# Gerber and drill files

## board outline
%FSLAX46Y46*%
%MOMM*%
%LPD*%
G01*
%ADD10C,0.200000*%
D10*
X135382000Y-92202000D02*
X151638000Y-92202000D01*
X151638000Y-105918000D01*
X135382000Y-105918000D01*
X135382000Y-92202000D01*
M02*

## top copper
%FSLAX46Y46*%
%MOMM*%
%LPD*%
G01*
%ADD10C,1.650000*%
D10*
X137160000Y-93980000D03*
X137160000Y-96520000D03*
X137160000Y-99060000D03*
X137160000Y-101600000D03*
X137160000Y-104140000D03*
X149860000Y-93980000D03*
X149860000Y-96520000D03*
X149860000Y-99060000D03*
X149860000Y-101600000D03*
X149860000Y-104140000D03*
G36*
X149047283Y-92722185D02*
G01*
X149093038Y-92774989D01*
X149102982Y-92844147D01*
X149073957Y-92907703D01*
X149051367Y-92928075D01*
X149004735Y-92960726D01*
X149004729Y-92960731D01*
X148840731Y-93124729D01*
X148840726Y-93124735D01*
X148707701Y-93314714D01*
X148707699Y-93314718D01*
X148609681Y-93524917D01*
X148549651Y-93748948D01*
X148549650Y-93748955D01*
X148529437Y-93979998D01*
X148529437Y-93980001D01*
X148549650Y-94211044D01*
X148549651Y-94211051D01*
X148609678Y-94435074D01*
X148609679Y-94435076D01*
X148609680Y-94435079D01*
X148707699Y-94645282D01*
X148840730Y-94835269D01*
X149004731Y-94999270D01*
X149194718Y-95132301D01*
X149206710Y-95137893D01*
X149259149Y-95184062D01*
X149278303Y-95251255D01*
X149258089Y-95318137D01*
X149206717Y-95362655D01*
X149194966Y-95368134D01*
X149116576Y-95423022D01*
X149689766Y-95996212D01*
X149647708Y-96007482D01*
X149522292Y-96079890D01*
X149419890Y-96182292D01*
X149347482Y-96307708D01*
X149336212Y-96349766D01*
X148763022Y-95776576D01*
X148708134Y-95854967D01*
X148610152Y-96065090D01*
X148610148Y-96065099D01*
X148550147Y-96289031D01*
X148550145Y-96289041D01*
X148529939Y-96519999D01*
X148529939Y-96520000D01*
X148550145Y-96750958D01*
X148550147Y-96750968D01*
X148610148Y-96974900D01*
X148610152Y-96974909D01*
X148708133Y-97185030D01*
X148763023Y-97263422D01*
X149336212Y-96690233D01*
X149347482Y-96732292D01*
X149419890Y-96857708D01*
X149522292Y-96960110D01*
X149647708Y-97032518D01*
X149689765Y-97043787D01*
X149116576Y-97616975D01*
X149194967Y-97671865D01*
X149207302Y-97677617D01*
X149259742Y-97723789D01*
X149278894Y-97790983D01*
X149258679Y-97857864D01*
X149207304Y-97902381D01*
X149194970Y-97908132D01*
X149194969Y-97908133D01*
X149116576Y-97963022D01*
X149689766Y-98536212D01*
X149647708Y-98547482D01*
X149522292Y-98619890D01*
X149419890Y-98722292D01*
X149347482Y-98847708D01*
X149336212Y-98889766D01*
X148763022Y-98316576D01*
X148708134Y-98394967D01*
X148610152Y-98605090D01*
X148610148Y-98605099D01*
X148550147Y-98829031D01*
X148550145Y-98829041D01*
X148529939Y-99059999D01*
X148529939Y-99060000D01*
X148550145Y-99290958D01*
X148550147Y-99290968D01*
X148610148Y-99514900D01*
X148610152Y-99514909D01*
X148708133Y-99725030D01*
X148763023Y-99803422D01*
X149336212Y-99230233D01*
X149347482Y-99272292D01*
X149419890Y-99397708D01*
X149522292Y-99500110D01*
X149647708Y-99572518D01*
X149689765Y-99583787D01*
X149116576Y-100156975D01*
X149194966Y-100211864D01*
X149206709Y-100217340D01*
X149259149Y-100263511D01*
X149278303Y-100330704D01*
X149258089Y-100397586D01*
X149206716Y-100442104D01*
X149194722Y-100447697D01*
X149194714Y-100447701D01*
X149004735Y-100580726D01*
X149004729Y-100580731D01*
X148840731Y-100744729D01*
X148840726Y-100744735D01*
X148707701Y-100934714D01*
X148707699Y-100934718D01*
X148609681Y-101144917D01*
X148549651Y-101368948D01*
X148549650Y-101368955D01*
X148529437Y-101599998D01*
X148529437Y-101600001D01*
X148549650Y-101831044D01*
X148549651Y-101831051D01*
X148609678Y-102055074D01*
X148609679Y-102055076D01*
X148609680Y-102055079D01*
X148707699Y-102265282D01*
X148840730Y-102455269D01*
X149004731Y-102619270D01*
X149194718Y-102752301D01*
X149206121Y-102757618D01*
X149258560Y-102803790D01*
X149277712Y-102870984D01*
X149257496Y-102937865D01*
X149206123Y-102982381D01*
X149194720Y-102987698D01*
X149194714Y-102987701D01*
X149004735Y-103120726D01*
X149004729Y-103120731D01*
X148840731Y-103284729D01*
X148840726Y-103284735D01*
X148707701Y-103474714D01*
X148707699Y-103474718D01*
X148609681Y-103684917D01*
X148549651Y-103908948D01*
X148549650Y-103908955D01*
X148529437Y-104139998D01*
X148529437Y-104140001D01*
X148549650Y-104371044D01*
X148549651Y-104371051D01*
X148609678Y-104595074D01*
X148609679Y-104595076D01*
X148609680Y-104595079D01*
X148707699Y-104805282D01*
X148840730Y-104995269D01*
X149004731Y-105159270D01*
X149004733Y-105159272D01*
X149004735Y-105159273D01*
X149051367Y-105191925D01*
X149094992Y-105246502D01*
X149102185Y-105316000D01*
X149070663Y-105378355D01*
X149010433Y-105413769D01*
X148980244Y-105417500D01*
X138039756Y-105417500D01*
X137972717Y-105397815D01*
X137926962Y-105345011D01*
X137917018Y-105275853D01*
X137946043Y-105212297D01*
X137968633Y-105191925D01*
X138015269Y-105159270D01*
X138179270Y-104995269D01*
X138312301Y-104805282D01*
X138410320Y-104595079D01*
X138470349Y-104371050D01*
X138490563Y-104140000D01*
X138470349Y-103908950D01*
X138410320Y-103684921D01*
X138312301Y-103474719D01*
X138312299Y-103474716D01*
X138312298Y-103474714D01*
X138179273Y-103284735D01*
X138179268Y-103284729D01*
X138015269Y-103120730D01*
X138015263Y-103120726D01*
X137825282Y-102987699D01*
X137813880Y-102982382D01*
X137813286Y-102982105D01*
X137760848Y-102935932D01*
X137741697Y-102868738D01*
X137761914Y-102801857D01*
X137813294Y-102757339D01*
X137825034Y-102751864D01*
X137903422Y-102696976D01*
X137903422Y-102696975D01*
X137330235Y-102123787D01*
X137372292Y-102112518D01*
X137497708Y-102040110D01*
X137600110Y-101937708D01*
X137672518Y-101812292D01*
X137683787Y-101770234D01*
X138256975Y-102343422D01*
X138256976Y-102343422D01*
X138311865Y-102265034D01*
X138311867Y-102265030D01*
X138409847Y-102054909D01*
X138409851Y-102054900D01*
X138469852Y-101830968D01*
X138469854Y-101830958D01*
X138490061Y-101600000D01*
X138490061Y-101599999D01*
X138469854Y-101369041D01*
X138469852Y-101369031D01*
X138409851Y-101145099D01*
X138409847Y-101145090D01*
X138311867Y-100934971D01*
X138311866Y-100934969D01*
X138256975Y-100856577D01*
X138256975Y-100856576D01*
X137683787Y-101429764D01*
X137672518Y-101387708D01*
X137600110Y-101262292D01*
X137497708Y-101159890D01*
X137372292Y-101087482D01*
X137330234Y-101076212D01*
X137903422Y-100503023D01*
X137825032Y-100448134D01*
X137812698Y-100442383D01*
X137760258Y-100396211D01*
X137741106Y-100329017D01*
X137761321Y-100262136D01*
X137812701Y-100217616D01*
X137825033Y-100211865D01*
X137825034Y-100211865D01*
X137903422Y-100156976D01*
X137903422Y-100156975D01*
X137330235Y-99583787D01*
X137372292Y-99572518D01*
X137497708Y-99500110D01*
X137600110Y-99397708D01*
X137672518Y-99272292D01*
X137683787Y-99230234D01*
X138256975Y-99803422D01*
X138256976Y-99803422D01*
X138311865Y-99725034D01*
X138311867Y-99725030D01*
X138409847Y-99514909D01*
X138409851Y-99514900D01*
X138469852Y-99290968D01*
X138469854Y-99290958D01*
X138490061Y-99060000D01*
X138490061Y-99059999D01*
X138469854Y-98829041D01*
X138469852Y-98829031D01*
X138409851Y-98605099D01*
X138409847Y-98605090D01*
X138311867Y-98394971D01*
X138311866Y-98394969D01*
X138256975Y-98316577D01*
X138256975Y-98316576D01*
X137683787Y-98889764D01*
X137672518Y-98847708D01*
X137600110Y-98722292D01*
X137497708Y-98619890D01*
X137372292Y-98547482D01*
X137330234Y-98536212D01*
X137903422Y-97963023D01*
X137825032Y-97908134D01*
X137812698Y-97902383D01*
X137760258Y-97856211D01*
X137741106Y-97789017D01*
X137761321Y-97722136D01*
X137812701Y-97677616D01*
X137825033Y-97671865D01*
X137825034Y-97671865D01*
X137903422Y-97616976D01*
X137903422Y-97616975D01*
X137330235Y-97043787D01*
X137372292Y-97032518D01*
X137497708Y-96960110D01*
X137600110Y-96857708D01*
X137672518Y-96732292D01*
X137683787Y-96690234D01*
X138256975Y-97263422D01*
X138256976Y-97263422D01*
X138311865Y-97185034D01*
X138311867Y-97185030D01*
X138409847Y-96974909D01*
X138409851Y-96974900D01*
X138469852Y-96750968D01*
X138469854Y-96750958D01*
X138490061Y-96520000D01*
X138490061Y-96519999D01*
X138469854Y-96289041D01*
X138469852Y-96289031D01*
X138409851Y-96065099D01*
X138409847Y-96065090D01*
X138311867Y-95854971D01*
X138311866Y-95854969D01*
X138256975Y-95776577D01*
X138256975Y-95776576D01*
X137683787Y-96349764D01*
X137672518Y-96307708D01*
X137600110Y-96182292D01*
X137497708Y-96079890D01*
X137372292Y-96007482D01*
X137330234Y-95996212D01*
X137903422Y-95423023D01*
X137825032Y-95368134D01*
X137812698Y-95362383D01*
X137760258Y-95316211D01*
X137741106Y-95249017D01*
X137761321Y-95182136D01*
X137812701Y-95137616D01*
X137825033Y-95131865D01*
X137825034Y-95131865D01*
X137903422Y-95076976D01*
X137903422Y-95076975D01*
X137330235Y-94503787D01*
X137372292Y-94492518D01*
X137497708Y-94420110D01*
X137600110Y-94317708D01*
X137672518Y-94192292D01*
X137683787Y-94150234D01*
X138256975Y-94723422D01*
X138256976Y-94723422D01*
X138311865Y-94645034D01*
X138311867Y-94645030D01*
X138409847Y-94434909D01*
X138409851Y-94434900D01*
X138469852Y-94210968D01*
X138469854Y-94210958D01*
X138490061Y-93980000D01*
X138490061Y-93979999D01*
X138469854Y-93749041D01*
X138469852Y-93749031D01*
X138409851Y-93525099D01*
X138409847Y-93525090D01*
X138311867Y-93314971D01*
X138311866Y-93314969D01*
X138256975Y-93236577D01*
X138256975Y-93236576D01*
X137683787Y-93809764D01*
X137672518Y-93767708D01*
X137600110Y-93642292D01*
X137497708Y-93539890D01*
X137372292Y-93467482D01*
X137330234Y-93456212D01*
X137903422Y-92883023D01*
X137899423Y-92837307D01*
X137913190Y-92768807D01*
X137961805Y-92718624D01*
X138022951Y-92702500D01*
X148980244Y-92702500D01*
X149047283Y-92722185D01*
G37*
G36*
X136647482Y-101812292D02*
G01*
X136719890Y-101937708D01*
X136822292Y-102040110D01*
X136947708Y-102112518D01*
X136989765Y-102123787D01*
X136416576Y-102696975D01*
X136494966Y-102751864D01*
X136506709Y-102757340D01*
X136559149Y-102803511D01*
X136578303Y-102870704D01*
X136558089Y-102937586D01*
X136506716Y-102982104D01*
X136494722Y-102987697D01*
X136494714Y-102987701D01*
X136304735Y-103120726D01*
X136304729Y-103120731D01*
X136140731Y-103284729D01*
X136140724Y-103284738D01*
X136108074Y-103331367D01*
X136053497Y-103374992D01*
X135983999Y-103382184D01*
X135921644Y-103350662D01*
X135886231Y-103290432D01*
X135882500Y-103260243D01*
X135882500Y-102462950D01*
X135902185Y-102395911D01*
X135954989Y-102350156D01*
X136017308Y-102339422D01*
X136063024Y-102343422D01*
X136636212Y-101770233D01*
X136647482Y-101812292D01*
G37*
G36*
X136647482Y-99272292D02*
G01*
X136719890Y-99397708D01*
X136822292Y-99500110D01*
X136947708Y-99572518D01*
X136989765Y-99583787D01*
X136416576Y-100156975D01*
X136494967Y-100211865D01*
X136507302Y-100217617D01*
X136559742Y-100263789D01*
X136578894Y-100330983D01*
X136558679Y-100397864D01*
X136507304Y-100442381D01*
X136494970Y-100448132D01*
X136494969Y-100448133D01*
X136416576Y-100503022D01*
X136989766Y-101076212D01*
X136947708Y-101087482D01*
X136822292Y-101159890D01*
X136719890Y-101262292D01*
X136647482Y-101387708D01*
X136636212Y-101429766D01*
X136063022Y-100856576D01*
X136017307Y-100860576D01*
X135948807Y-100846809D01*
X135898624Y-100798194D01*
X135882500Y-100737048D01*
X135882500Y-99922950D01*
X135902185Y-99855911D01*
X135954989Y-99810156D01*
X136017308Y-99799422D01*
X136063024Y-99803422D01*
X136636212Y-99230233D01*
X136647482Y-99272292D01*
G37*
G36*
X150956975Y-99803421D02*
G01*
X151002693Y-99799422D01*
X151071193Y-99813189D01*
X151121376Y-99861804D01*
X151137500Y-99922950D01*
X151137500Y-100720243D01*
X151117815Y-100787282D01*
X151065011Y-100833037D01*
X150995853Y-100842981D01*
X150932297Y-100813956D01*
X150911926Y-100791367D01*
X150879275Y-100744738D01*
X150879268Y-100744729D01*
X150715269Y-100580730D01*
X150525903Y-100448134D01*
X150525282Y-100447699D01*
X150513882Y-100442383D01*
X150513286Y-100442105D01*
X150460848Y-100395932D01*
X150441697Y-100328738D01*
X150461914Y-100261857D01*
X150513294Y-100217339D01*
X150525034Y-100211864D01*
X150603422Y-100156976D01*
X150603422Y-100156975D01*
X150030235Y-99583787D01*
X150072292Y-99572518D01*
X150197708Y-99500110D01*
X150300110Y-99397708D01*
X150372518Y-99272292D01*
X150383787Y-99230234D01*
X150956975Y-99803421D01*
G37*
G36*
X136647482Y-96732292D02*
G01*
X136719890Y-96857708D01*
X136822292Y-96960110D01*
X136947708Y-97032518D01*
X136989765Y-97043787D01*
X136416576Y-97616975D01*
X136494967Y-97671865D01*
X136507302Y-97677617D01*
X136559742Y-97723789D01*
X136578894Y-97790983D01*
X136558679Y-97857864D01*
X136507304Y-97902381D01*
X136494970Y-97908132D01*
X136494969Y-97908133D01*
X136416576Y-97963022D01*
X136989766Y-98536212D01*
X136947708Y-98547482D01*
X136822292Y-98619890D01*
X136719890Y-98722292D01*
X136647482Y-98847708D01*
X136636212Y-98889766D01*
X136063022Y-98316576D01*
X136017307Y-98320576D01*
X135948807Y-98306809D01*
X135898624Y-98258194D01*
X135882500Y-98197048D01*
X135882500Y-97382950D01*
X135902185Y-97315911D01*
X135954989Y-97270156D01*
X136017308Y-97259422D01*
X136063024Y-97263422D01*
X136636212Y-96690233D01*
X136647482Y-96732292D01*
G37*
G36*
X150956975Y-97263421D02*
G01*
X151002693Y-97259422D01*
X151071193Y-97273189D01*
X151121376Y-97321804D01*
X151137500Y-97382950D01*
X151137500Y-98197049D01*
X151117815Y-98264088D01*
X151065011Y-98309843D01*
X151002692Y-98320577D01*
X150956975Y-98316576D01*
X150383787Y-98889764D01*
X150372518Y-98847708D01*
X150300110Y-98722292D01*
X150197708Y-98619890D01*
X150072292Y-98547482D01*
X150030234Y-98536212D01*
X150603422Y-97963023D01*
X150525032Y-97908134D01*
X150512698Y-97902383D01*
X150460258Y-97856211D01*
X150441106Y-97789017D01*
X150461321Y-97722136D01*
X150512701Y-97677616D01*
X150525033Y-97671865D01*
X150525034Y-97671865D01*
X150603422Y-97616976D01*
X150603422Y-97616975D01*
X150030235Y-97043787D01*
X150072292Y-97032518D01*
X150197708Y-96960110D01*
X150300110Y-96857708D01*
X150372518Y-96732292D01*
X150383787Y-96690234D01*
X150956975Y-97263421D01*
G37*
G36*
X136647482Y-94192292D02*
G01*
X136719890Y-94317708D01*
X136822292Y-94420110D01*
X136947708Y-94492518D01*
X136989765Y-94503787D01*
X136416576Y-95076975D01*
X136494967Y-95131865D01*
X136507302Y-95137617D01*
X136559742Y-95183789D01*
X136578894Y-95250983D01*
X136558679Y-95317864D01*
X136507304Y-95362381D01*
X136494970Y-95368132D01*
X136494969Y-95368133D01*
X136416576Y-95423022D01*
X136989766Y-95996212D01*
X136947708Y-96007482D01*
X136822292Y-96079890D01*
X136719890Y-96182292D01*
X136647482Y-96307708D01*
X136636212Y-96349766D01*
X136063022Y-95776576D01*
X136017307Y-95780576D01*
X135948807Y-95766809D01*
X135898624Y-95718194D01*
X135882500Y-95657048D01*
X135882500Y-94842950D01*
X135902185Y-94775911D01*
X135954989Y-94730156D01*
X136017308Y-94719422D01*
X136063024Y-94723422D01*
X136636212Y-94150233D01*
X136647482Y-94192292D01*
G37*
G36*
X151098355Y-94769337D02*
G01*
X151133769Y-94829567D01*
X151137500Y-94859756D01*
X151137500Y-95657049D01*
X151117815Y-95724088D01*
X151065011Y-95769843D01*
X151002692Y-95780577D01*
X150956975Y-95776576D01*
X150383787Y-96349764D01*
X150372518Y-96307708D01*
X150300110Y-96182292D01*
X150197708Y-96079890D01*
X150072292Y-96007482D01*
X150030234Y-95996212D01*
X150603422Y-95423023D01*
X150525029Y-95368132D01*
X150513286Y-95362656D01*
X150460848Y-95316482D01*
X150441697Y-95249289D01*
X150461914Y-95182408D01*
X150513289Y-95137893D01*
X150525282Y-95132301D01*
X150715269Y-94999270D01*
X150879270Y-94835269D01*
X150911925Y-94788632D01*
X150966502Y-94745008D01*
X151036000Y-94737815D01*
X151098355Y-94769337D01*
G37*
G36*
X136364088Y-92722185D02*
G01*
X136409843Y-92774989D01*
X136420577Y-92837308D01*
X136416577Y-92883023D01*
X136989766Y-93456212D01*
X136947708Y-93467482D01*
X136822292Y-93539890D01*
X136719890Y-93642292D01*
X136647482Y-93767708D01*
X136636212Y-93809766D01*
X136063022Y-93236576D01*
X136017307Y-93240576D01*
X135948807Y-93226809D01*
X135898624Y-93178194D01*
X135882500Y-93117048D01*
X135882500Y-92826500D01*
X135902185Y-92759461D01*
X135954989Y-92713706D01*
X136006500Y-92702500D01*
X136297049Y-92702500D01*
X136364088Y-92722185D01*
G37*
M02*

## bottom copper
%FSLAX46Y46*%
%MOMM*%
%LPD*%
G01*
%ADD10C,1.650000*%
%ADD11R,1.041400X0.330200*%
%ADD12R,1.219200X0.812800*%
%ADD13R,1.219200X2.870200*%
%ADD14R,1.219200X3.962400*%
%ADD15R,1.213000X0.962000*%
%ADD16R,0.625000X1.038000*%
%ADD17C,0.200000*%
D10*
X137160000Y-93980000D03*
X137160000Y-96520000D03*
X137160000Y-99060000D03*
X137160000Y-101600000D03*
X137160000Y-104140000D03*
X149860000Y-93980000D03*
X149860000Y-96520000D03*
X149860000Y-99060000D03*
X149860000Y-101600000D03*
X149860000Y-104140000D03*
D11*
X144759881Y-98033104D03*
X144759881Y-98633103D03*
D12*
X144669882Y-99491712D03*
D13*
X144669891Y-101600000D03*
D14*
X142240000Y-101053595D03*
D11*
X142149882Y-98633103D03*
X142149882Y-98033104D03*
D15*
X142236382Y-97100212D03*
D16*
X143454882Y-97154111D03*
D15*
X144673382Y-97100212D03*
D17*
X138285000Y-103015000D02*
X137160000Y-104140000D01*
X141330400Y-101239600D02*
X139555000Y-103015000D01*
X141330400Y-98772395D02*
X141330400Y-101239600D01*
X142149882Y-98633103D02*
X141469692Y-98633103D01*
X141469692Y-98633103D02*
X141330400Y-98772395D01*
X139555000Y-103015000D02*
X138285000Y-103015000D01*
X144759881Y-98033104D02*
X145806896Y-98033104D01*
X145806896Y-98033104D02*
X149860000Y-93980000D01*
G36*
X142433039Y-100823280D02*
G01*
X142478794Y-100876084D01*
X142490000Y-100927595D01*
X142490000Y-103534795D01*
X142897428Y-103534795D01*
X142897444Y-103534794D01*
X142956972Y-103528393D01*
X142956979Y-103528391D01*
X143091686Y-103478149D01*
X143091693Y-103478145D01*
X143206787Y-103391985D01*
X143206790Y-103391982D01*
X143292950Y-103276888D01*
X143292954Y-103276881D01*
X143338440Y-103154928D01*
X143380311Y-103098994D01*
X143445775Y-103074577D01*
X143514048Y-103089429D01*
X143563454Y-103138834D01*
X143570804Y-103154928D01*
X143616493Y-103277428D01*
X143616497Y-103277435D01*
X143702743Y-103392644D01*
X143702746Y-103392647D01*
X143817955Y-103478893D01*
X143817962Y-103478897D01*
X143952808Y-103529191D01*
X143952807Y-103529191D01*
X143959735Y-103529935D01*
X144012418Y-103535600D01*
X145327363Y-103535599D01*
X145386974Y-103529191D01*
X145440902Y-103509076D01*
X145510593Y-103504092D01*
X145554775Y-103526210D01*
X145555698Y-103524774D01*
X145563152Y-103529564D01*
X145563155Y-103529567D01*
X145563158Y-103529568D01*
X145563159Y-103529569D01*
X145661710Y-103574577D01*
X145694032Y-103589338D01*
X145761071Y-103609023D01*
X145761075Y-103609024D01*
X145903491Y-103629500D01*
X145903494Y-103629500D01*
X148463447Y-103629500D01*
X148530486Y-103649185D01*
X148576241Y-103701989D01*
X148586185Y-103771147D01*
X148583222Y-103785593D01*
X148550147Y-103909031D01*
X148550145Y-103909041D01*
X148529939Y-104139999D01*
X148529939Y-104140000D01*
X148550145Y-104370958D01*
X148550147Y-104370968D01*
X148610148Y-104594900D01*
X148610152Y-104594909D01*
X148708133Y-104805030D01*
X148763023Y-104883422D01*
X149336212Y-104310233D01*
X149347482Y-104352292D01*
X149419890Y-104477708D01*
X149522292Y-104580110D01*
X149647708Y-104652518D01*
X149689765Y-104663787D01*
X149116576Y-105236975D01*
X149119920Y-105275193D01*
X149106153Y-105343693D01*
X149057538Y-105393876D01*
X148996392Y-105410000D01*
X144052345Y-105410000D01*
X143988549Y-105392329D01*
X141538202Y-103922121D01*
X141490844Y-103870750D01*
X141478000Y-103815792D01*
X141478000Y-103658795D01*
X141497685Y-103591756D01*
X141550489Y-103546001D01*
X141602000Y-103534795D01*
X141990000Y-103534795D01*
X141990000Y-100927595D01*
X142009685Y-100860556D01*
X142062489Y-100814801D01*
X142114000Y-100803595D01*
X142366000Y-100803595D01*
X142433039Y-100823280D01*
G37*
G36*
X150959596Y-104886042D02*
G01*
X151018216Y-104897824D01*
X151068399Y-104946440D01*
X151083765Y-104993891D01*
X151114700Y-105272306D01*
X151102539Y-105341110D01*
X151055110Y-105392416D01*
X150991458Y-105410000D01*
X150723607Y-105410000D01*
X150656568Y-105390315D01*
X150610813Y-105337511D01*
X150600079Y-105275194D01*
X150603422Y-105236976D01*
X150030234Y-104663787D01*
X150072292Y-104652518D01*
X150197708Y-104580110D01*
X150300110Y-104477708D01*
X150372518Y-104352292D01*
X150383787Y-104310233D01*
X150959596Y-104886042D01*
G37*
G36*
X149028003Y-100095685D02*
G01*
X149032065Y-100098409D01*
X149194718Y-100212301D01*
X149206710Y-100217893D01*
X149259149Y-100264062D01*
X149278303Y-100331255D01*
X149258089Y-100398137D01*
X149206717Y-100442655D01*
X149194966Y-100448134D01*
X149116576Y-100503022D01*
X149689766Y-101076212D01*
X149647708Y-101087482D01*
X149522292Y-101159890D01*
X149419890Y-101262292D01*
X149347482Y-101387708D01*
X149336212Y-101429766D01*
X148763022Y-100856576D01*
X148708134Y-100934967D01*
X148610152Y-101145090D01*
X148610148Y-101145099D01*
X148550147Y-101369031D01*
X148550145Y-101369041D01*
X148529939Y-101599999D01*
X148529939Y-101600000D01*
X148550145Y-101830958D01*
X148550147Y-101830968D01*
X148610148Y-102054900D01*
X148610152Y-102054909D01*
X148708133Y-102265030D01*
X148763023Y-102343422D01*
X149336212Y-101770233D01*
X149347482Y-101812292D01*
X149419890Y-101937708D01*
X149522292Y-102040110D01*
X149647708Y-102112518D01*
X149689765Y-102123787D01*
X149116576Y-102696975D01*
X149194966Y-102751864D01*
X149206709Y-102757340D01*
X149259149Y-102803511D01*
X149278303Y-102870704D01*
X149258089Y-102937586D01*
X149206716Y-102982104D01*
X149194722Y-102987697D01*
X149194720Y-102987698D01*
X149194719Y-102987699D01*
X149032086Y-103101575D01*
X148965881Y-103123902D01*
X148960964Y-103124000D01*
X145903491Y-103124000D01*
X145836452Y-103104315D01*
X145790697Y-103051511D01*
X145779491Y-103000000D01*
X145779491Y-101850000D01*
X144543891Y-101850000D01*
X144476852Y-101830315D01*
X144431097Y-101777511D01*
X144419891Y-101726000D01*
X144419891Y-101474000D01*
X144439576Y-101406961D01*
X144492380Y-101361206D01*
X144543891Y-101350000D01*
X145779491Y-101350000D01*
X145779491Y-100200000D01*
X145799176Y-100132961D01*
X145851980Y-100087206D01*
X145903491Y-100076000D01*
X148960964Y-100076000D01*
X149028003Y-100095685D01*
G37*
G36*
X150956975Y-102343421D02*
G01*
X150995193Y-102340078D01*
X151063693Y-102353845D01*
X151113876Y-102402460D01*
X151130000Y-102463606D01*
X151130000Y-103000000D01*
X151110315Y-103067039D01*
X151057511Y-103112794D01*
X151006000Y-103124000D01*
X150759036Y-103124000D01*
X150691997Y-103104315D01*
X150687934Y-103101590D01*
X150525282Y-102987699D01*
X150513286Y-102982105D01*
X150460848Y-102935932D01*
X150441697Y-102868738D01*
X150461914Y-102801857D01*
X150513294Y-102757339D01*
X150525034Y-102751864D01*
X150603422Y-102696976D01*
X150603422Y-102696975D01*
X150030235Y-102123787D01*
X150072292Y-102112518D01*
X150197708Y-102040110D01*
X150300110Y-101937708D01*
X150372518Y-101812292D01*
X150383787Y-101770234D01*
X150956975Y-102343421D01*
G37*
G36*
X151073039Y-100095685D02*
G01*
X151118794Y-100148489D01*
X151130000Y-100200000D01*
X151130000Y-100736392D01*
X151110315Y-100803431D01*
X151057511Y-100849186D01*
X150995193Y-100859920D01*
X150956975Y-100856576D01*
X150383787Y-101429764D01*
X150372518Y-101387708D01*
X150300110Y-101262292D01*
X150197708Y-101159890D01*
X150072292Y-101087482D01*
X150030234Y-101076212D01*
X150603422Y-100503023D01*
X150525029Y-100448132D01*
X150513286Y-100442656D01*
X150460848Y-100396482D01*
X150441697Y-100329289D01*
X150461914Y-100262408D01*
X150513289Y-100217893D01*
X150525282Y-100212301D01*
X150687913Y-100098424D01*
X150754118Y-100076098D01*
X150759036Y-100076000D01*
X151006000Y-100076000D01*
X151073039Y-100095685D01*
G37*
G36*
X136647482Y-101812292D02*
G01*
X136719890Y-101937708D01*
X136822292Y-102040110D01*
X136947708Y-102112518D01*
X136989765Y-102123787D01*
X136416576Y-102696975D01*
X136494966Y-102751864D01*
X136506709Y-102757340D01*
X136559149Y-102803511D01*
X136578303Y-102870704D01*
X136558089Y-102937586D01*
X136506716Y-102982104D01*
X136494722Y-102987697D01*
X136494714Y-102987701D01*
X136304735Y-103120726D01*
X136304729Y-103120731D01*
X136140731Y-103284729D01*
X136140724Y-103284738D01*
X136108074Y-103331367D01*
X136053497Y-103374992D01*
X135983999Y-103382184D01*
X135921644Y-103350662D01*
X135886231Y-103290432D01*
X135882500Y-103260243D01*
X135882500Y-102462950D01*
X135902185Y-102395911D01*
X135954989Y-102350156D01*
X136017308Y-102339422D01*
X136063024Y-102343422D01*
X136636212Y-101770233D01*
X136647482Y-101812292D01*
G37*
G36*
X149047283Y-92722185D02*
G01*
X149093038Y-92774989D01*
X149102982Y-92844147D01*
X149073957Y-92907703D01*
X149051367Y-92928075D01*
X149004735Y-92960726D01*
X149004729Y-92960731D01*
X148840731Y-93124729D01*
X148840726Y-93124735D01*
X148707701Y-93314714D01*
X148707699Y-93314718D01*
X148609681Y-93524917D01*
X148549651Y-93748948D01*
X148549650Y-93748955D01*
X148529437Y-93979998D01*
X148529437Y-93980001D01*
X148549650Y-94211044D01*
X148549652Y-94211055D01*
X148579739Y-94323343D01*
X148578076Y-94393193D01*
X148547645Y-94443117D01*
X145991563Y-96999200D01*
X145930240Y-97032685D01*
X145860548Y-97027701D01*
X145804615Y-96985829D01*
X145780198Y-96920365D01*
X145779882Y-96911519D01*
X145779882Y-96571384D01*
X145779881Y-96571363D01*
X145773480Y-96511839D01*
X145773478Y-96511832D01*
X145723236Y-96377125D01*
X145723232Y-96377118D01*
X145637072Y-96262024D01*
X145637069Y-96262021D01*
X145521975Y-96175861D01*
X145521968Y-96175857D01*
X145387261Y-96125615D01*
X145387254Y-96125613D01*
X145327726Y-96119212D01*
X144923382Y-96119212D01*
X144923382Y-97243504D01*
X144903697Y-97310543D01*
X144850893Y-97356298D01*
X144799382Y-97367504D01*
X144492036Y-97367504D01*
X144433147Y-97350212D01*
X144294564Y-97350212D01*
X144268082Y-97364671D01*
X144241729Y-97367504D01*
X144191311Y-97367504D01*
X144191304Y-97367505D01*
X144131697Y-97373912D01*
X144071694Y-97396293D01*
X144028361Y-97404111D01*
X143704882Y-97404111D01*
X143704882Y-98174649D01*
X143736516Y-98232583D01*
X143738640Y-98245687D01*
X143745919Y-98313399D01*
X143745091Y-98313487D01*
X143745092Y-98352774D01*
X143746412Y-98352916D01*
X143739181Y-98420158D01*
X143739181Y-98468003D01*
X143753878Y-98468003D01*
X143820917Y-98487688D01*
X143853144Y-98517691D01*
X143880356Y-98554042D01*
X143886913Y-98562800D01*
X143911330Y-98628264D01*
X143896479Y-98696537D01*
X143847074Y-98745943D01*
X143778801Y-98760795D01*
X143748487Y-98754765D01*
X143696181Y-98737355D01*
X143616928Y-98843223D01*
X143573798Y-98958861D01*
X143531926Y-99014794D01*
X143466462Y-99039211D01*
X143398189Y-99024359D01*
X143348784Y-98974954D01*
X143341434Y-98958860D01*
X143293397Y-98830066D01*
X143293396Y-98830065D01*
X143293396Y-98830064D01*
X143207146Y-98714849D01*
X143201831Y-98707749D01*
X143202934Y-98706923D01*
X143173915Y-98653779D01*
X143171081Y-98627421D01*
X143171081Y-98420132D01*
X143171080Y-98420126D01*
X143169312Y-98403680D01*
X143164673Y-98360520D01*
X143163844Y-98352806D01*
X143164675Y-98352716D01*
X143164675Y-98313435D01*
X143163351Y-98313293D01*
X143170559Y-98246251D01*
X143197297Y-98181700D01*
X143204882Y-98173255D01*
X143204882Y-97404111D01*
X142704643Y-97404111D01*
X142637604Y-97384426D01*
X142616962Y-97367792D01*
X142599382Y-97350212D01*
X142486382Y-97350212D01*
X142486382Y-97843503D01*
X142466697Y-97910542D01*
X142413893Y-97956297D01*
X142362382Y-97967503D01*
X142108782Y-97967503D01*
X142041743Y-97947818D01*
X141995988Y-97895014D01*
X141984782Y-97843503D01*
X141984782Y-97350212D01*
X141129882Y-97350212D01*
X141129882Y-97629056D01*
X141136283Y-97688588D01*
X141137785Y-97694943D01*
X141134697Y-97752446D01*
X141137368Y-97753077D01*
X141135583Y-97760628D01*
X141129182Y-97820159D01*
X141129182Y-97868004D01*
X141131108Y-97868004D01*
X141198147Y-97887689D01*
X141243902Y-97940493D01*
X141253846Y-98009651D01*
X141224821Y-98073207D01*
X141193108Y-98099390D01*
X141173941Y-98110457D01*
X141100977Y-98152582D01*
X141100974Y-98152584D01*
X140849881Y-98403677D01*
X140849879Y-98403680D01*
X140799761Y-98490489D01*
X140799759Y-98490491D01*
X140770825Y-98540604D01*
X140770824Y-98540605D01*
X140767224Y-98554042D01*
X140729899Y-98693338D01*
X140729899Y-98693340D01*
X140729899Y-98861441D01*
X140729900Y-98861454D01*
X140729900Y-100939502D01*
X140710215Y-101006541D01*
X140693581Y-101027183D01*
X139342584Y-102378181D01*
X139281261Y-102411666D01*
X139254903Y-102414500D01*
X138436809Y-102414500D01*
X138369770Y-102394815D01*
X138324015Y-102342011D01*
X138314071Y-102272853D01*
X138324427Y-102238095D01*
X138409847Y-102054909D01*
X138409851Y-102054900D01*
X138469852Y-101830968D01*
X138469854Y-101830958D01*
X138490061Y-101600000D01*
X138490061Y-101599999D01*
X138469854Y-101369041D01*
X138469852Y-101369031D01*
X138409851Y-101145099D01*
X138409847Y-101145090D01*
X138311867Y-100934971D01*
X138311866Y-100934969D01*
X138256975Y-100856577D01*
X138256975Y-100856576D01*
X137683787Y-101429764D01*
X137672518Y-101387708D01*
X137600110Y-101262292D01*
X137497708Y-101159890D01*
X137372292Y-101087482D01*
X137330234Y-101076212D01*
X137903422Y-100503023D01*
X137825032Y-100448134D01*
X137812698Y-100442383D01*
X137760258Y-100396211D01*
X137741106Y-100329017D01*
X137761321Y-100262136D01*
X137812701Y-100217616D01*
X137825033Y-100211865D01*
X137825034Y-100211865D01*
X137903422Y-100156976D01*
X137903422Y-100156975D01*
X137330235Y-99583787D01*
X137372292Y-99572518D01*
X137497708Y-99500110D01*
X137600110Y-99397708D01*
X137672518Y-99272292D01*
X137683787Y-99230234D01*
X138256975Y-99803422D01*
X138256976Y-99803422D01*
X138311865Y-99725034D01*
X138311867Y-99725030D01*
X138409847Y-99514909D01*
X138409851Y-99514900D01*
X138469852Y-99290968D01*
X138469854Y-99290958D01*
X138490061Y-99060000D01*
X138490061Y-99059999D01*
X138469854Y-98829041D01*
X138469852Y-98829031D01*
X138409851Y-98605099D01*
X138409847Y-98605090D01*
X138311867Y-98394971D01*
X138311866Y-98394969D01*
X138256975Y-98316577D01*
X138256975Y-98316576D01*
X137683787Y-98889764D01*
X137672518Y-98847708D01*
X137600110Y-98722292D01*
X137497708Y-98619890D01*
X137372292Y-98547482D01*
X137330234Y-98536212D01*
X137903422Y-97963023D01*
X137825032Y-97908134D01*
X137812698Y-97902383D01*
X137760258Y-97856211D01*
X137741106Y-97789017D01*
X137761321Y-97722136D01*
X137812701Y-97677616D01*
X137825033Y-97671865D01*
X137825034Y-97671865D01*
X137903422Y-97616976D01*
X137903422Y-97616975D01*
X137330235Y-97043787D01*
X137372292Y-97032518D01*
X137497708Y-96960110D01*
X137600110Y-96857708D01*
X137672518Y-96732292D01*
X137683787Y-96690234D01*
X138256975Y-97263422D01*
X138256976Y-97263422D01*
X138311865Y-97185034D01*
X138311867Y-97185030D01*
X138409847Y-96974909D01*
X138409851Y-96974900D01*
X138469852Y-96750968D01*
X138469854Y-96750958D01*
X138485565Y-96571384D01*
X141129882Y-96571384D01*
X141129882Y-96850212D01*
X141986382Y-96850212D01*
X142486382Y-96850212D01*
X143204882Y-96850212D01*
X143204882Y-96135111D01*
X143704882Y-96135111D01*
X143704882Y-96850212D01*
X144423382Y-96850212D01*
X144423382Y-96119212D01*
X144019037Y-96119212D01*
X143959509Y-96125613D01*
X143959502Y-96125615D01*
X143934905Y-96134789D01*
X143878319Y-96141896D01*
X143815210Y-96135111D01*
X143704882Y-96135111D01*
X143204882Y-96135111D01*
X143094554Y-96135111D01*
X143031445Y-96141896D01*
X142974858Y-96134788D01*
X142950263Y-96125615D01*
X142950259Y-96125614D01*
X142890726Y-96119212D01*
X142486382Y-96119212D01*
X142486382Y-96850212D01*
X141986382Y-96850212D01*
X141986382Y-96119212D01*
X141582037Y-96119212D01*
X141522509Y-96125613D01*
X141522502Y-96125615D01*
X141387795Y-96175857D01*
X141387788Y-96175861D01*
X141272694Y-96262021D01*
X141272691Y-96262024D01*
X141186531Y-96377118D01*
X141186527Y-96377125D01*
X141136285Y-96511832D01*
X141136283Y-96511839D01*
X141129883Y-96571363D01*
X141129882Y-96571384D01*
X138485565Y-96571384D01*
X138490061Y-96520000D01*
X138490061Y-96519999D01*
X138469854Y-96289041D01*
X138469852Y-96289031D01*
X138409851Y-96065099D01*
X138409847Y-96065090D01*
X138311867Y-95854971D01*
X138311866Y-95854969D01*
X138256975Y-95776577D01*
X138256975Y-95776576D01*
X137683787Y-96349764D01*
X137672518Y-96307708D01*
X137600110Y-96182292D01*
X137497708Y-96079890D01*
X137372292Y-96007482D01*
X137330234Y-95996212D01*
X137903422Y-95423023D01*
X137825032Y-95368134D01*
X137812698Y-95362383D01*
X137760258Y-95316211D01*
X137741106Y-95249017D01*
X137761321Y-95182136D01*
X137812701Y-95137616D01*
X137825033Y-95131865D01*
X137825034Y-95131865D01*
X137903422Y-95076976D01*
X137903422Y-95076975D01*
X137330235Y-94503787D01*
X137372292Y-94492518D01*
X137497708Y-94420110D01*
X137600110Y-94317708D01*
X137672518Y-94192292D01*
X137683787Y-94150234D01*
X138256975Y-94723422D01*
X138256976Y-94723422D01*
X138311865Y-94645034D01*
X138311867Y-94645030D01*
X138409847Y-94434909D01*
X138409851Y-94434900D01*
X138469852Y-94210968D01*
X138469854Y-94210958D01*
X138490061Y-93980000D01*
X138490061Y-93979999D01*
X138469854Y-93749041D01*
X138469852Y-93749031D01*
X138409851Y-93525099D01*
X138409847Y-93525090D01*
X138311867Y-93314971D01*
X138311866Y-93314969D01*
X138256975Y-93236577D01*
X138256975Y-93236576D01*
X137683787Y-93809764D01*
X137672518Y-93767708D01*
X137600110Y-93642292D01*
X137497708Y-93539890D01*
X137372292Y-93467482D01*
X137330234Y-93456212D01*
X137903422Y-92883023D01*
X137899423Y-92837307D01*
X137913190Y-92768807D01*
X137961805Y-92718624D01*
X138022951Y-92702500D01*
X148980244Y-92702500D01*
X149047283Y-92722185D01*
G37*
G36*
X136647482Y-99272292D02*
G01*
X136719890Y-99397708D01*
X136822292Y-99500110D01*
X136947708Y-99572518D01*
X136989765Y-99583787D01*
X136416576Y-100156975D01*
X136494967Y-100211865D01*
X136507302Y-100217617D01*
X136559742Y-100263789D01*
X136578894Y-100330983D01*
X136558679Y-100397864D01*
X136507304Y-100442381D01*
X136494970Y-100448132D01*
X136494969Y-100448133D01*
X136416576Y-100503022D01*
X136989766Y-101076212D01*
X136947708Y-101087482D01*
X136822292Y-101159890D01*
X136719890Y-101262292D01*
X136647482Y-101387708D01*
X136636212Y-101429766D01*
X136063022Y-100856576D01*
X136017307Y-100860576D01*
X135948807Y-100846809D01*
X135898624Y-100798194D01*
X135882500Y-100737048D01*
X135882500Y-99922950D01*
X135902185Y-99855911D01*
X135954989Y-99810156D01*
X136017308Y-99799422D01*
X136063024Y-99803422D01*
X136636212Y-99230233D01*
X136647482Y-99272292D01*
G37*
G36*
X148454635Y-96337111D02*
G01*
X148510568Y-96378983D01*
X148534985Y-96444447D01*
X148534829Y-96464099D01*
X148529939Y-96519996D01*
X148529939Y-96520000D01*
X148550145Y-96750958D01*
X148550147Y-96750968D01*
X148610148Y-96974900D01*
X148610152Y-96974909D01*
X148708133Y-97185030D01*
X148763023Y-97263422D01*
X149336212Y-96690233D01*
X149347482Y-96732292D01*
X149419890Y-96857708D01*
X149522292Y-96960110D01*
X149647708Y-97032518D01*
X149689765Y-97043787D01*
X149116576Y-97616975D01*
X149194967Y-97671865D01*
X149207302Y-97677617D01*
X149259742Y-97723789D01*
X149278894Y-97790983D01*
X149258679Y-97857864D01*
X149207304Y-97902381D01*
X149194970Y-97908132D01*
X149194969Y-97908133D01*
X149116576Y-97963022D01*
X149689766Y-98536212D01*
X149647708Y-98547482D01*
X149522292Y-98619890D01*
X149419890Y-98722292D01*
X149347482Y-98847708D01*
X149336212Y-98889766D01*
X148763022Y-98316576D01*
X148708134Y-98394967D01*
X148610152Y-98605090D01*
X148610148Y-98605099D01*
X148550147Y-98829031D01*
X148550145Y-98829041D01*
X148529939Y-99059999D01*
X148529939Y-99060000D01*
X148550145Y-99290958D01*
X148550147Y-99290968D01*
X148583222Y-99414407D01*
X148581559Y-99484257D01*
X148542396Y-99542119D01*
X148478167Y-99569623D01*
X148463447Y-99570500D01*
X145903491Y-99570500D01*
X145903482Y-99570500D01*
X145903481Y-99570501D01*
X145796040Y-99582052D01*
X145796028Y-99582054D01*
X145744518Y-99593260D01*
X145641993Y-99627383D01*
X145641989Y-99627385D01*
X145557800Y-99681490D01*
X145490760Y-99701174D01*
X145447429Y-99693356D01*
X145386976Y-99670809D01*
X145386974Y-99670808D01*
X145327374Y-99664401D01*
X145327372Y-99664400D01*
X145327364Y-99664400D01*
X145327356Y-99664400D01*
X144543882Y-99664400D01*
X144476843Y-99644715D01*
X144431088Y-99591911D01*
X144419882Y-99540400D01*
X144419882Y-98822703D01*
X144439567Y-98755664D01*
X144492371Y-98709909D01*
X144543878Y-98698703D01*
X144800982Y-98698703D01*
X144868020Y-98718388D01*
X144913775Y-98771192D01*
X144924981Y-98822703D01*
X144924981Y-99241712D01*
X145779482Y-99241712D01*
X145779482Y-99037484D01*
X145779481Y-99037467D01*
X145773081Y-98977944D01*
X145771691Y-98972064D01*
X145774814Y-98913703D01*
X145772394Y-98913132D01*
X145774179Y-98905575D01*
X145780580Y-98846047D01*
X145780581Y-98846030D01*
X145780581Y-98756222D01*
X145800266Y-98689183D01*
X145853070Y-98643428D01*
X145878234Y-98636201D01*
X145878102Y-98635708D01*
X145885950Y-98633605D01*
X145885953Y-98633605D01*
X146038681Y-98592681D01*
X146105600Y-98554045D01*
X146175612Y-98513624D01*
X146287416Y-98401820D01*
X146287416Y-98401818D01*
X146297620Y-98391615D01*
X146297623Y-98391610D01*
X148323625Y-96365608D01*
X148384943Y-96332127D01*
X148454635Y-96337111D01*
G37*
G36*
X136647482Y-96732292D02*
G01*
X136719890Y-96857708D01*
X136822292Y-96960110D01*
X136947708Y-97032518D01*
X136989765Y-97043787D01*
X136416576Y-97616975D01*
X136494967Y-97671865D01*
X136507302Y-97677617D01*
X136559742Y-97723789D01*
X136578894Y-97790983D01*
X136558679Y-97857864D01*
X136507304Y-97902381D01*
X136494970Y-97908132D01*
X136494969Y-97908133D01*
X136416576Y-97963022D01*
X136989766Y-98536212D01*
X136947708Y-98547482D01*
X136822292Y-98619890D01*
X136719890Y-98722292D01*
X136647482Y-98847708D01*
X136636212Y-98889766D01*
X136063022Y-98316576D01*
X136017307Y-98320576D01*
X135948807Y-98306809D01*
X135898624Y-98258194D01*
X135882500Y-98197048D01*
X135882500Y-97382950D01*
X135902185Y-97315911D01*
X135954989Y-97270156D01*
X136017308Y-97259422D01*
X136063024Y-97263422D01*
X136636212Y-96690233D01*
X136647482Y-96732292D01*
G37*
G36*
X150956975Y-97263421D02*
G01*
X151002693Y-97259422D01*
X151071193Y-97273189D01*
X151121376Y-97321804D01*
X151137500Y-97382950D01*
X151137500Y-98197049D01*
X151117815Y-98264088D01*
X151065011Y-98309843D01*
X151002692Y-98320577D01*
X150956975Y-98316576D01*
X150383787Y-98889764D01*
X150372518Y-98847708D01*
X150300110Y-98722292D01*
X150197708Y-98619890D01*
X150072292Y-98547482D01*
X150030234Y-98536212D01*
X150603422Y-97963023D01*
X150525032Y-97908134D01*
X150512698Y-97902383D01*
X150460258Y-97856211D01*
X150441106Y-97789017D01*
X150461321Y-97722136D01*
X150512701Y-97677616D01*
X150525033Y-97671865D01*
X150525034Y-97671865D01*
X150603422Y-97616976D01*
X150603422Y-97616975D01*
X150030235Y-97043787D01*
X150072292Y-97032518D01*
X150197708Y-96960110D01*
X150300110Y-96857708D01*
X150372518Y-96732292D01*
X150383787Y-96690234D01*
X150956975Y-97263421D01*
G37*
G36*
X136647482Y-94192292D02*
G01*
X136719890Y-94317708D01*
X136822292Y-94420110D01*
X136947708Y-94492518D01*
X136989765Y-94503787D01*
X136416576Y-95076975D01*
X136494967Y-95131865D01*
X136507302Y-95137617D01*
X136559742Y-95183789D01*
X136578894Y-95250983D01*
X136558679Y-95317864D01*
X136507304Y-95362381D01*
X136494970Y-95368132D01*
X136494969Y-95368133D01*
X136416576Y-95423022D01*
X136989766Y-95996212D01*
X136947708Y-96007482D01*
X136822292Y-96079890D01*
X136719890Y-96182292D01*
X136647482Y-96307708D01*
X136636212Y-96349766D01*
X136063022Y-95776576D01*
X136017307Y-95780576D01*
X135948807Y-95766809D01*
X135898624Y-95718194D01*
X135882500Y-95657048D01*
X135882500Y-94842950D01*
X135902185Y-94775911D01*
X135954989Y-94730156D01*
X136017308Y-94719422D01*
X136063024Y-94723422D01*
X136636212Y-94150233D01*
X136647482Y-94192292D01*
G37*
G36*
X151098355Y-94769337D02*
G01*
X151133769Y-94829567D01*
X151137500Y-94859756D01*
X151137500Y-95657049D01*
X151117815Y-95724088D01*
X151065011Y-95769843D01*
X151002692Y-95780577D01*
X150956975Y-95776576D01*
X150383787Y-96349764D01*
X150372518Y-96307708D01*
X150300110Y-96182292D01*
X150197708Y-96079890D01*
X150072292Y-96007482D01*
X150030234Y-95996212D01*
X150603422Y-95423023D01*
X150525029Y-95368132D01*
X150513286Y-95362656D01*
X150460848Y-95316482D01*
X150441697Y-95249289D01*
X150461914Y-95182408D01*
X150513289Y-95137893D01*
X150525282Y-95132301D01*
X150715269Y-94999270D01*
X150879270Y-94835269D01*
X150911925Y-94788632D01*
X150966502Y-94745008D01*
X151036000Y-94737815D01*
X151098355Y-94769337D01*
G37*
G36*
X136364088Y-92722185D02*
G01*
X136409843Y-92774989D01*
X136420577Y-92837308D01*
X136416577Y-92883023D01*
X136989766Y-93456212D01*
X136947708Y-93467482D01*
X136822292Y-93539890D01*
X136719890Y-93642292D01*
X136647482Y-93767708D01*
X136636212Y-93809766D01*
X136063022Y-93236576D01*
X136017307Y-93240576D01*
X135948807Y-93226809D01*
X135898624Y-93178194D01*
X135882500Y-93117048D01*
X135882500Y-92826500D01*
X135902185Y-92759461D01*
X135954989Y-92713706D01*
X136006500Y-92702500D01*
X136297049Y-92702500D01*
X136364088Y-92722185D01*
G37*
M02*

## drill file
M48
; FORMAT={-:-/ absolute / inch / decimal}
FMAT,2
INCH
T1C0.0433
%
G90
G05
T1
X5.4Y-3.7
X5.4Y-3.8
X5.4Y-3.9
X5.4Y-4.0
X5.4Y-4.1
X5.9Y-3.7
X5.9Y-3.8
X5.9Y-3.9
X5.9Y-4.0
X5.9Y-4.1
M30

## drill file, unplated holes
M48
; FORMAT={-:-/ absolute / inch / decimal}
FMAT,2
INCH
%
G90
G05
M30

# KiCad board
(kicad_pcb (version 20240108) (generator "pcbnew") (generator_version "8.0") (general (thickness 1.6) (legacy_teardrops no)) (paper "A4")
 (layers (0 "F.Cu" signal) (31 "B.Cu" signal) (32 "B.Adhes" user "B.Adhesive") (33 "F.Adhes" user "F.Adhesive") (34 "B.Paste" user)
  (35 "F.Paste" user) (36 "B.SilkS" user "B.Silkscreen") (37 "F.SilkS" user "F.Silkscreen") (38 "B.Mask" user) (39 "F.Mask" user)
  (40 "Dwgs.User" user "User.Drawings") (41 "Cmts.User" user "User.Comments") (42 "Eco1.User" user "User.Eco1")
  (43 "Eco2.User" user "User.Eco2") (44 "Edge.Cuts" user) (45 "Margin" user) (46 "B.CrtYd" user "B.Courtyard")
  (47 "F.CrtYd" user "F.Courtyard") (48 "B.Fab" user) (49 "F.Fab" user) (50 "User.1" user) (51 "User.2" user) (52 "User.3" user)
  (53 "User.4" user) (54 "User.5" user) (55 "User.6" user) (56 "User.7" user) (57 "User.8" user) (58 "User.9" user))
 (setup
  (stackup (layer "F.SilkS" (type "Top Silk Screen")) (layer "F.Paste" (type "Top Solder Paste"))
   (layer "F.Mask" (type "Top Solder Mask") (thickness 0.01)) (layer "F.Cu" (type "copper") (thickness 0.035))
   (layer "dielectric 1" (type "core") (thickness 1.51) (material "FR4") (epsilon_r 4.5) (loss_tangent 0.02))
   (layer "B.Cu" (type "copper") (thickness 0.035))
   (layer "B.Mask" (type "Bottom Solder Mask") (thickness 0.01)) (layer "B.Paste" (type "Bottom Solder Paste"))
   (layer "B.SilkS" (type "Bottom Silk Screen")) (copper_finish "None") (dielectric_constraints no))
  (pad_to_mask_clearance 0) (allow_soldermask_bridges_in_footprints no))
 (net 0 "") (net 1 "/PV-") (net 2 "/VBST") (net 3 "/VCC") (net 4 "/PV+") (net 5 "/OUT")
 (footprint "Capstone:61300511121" (layer "F.Cu") (at 137.16 99.06 -90)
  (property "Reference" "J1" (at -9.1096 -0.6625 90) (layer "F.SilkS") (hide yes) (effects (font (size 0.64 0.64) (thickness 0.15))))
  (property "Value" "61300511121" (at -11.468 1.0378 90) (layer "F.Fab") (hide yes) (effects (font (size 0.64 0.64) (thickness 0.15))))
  (pad "1" thru_hole circle (at -5.08 0 270) (size 1.65 1.65) (drill 1.1) (layers "*.Cu" "*.Mask") (remove_unused_layers no) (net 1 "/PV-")
   (solder_mask_margin 0.102))
  (pad "2" thru_hole circle (at -2.54 0 270) (size 1.65 1.65) (drill 1.1) (layers "*.Cu" "*.Mask") (remove_unused_layers no) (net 1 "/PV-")
   (solder_mask_margin 0.102))
  (pad "3" thru_hole circle (at 0 0 270) (size 1.65 1.65) (drill 1.1) (layers "*.Cu" "*.Mask") (remove_unused_layers no) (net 1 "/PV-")
   (solder_mask_margin 0.102))
  (pad "4" thru_hole circle (at 2.54 0 270) (size 1.65 1.65) (drill 1.1) (layers "*.Cu" "*.Mask") (remove_unused_layers no) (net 1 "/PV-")
   (solder_mask_margin 0.102))
  (pad "5" thru_hole circle (at 5.08 0 270) (size 1.65 1.65) (drill 1.1) (layers "*.Cu" "*.Mask") (remove_unused_layers no) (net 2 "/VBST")
   (solder_mask_margin 0.102)))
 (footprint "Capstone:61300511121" (layer "F.Cu") (at 149.86 99.06 -90)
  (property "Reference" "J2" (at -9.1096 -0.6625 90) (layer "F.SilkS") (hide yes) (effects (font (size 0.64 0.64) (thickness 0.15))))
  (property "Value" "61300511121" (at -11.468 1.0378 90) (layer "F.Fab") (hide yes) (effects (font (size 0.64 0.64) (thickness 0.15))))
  (pad "1" thru_hole circle (at -5.08 0 270) (size 1.65 1.65) (drill 1.1) (layers "*.Cu" "*.Mask") (remove_unused_layers no) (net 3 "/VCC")
   (solder_mask_margin 0.102))
  (pad "2" thru_hole circle (at -2.54 0 270) (size 1.65 1.65) (drill 1.1) (layers "*.Cu" "*.Mask") (remove_unused_layers no) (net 1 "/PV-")
   (solder_mask_margin 0.102))
  (pad "3" thru_hole circle (at 0 0 270) (size 1.65 1.65) (drill 1.1) (layers "*.Cu" "*.Mask") (remove_unused_layers no) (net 1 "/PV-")
   (solder_mask_margin 0.102))
  (pad "4" thru_hole circle (at 2.54 0 270) (size 1.65 1.65) (drill 1.1) (layers "*.Cu" "*.Mask") (remove_unused_layers no) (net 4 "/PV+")
   (solder_mask_margin 0.102))
  (pad "5" thru_hole circle (at 5.08 0 270) (size 1.65 1.65) (drill 1.1) (layers "*.Cu" "*.Mask") (remove_unused_layers no) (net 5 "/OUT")
   (solder_mask_margin 0.102)))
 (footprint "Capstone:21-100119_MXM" (layer "B.Cu") (at 142.149882 98.633103 180)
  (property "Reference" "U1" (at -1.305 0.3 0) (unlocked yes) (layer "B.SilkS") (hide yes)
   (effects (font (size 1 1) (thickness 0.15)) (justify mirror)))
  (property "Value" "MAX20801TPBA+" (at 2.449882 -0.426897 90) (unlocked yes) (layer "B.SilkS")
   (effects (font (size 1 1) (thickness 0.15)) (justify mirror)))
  (pad "1" smd rect (at -2.609999 0.599999 180) (size 1.0414 0.3302) (layers "B.Cu" "B.Paste" "B.Mask") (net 3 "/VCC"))
  (pad "2" smd rect (at -2.609999 0 180) (size 1.0414 0.3302) (layers "B.Cu" "B.Paste" "B.Mask") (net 1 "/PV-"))
  (pad "3" smd rect (at -2.52 -0.858609 180) (size 1.2192 0.8128) (layers "B.Cu" "B.Paste" "B.Mask") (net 1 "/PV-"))
  (pad "4" smd rect (at -2.520009 -2.966897 180) (size 1.2192 2.8702) (layers "B.Cu" "B.Paste" "B.Mask") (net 4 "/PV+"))
  (pad "5" smd rect (at -0.090118 -2.420492 180) (size 1.2192 3.9624) (layers "B.Cu" "B.Paste" "B.Mask") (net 5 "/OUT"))
  (pad "6" smd rect (at 0 0 180) (size 1.0414 0.3302) (layers "B.Cu" "B.Paste" "B.Mask") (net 2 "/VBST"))
  (pad "7" smd rect (at 0 0.599999 180) (size 1.0414 0.3302) (layers "B.Cu" "B.Paste" "B.Mask") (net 1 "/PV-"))
  (pad "8" smd rect (at -0.0865 1.532891 180) (size 1.213 0.962) (layers "B.Cu" "B.Paste" "B.Mask") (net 1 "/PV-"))
  (pad "9" smd rect (at -1.305 1.478992 180) (size 0.625 1.038) (layers "B.Cu" "B.Paste" "B.Mask") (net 1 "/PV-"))
  (pad "10" smd rect (at -2.5235 1.532891 180) (size 1.213 0.962) (layers "B.Cu" "B.Paste" "B.Mask") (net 1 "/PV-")))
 (gr_rect (start 135.382 92.202) (end 151.638 105.918) (stroke (width 0.2) (type default)) (fill none) (layer "Edge.Cuts"))
 (segment (start 142.149882 98.633103) (end 141.469692 98.633103) (width 0.2) (layer "B.Cu") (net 2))
 (segment (start 141.3304 101.2396) (end 139.555 103.015) (width 0.2) (layer "B.Cu") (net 2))
 (segment (start 141.469692 98.633103) (end 141.3304 98.772395) (width 0.2) (layer "B.Cu") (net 2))
 (segment (start 138.285 103.015) (end 137.16 104.14) (width 0.2) (layer "B.Cu") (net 2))
 (segment (start 139.555 103.015) (end 138.285 103.015) (width 0.2) (layer "B.Cu") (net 2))
 (segment (start 141.3304 98.772395) (end 141.3304 101.2396) (width 0.2) (layer "B.Cu") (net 2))
 (segment (start 144.759881 98.033104) (end 145.806896 98.033104) (width 0.2) (layer "B.Cu") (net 3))
 (segment (start 145.806896 98.033104) (end 149.86 93.98) (width 0.2) (layer "B.Cu") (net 3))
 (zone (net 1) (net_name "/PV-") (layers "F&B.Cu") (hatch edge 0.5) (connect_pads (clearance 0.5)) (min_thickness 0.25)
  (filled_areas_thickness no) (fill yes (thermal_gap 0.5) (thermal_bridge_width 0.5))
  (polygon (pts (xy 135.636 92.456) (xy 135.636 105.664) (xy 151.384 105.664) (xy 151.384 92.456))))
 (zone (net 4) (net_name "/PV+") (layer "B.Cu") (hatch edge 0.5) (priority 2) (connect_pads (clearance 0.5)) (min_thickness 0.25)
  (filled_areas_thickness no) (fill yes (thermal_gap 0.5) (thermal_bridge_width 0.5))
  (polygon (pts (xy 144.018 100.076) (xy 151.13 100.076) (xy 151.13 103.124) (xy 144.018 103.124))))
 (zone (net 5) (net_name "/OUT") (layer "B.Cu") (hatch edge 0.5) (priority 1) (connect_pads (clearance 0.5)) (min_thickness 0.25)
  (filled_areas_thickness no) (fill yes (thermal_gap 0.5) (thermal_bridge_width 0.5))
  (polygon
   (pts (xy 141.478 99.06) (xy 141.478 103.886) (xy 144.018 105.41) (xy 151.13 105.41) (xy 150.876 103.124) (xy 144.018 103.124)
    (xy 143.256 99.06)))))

